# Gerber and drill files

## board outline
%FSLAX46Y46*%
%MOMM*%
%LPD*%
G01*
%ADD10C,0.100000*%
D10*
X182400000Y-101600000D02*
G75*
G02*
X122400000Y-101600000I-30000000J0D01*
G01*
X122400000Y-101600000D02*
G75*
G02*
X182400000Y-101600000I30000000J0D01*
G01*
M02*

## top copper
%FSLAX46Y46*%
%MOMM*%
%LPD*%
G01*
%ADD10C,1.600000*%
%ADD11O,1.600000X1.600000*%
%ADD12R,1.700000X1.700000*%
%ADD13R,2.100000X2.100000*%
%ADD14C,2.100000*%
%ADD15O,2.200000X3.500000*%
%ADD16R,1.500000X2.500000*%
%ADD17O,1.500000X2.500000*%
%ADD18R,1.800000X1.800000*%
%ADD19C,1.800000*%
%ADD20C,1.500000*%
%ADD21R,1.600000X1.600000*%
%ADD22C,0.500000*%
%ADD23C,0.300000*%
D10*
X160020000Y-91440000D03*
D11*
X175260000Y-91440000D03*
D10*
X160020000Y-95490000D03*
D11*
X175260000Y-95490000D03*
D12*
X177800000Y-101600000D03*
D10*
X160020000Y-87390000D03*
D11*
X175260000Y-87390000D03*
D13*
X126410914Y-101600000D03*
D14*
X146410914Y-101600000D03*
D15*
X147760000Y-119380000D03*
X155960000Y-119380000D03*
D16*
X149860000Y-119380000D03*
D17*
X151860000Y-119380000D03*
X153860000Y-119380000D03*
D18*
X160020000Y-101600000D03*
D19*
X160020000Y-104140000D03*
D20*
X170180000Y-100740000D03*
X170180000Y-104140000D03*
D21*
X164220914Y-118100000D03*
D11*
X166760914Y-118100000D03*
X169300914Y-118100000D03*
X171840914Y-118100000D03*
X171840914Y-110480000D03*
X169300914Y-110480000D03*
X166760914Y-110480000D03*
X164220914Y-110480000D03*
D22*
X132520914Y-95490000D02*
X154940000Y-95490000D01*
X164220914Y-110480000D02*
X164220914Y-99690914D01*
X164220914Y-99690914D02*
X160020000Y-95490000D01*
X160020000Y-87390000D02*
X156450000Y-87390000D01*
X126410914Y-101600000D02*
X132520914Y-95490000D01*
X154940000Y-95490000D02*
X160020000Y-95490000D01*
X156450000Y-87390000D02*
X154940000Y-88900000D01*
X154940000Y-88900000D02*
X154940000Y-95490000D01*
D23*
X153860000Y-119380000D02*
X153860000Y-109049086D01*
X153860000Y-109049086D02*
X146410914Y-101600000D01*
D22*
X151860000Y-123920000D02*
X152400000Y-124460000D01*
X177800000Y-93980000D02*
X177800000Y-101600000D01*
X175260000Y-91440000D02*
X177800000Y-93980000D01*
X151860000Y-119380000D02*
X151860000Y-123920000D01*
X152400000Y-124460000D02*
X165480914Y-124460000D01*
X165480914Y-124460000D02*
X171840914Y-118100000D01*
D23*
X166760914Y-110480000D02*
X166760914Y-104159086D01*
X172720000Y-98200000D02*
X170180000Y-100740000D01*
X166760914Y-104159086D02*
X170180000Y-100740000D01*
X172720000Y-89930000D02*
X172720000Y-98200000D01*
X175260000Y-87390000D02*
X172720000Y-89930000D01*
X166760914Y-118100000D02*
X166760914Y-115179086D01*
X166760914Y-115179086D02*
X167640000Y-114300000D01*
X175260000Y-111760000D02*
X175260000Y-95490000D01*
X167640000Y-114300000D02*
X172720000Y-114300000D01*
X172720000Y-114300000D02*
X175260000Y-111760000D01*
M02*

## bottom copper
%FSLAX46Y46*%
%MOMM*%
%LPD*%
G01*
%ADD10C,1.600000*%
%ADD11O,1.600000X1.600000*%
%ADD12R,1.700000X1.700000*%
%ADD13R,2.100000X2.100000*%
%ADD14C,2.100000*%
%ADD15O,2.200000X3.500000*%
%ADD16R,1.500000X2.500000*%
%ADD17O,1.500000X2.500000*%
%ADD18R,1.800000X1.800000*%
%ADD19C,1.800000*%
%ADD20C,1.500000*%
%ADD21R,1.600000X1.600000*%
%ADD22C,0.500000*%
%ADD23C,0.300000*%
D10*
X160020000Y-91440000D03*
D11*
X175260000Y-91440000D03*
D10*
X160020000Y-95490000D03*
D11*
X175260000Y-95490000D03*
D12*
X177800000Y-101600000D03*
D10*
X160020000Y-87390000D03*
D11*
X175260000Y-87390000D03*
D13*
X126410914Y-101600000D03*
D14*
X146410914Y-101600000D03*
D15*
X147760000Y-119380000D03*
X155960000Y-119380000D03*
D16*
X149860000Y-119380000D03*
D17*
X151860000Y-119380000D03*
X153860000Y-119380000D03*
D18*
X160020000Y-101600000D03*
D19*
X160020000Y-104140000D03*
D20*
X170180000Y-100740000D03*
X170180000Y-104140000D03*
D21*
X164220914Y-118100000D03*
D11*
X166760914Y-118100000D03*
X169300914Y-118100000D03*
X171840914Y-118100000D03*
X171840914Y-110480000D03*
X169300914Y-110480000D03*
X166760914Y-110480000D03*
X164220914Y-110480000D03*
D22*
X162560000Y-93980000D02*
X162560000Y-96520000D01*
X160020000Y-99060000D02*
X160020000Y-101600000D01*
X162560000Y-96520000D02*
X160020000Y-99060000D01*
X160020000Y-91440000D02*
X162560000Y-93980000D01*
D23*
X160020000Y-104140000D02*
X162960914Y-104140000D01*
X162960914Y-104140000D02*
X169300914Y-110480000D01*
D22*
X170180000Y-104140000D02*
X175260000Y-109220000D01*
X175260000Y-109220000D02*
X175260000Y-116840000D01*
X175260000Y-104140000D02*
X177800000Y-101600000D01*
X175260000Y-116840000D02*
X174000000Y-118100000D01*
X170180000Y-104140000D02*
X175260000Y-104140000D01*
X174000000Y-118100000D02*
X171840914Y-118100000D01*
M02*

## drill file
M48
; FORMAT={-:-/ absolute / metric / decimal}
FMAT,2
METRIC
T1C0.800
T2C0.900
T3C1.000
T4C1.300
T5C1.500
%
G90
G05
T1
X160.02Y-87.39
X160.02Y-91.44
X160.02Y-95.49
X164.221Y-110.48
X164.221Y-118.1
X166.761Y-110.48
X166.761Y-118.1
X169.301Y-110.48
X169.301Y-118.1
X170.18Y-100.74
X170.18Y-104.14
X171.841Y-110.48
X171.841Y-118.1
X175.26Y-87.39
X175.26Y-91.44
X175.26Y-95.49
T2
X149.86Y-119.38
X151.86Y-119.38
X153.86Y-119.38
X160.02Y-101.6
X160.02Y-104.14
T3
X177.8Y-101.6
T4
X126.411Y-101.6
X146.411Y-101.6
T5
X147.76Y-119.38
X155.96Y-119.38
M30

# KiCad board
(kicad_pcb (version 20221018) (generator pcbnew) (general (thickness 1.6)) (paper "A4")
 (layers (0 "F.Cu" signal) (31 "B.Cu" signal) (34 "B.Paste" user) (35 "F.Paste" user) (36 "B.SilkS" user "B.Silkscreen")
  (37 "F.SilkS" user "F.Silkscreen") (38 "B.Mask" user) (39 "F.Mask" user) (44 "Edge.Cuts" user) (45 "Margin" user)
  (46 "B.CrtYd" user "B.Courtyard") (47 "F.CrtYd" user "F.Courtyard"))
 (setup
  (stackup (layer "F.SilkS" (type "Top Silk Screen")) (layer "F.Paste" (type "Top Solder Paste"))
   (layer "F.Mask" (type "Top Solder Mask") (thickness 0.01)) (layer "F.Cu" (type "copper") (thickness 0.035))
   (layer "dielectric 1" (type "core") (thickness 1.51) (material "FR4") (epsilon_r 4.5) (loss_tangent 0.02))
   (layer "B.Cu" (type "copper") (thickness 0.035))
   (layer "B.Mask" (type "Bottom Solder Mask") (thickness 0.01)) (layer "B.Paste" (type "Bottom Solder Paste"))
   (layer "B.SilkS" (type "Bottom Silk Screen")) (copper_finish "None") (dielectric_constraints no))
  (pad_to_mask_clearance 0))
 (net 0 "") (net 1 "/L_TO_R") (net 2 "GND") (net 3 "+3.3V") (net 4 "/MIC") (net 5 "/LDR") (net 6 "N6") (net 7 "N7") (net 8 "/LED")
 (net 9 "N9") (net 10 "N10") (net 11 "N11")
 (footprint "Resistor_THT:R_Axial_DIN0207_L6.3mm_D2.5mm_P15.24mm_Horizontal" (layer "F.Cu") (at 160.02 91.44)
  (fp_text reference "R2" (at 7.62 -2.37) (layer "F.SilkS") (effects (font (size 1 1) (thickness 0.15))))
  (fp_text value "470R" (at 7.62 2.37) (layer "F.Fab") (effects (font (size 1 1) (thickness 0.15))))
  (pad "1" thru_hole circle (at 0 0) (size 1.6 1.6) (drill 0.8) (layers "*.Cu" "*.Mask") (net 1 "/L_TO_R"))
  (pad "2" thru_hole oval (at 15.24 0) (size 1.6 1.6) (drill 0.8) (layers "*.Cu" "*.Mask") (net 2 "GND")))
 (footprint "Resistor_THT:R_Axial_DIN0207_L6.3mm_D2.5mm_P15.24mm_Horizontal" (layer "F.Cu") (at 160.02 95.49)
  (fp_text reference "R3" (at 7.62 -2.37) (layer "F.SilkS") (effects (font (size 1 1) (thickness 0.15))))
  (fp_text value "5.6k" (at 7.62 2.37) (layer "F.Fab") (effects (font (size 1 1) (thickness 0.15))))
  (pad "1" thru_hole circle (at 0 0) (size 1.6 1.6) (drill 0.8) (layers "*.Cu" "*.Mask") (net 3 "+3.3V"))
  (pad "2" thru_hole oval (at 15.24 0) (size 1.6 1.6) (drill 0.8) (layers "*.Cu" "*.Mask") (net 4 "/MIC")))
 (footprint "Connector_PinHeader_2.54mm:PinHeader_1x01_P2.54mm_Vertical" (layer "F.Cu") (at 177.8 101.6 90)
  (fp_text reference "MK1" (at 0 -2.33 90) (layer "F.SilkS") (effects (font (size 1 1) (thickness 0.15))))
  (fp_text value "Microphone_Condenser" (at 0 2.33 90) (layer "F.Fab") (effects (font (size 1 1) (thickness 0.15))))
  (pad "1" thru_hole rect (at 0 0 90) (size 1.7 1.7) (drill 1) (layers "*.Cu" "*.Mask") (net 2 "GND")))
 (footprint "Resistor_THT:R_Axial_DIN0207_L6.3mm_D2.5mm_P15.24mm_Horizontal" (layer "F.Cu") (at 160.02 87.39)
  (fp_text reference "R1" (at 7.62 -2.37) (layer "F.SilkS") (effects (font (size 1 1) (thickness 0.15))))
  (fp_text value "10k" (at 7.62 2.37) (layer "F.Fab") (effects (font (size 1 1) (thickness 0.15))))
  (pad "1" thru_hole circle (at 0 0) (size 1.6 1.6) (drill 0.8) (layers "*.Cu" "*.Mask") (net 3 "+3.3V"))
  (pad "2" thru_hole oval (at 15.24 0) (size 1.6 1.6) (drill 0.8) (layers "*.Cu" "*.Mask") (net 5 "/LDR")))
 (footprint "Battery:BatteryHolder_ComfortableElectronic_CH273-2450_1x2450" (layer "F.Cu") (at 126.410914 101.6)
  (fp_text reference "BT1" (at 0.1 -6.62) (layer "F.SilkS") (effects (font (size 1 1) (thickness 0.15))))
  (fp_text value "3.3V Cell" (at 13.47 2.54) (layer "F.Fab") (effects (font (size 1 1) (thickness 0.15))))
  (pad "1" thru_hole rect (at 0 0 270) (size 2.1 2.1) (drill 1.3) (layers "*.Cu" "*.Mask") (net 3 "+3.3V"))
  (pad "2" thru_hole circle (at 20 0 270) (size 2.1 2.1) (drill 1.3) (layers "*.Cu" "*.Mask") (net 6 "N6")))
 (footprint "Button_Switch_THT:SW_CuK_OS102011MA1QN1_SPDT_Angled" (layer "F.Cu") (at 149.86 119.38)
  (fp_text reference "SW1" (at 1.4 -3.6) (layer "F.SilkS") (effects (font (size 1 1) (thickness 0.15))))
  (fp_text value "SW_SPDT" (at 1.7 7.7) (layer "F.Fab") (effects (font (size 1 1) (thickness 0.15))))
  (pad "" thru_hole oval (at -2.1 0) (size 2.2 3.5) (drill 1.5) (layers "*.Cu" "*.Mask"))
  (pad "" thru_hole oval (at 6.1 0) (size 2.2 3.5) (drill 1.5) (layers "*.Cu" "*.Mask"))
  (pad "1" thru_hole rect (at 0 0) (size 1.5 2.5) (drill 0.9) (layers "*.Cu" "*.Mask") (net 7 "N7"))
  (pad "2" thru_hole oval (at 2 0) (size 1.5 2.5) (drill 0.9) (layers "*.Cu" "*.Mask") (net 2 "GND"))
  (pad "3" thru_hole oval (at 4 0) (size 1.5 2.5) (drill 0.9) (layers "*.Cu" "*.Mask") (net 6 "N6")))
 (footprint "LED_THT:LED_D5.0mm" (layer "F.Cu") (at 160.02 101.6 -90)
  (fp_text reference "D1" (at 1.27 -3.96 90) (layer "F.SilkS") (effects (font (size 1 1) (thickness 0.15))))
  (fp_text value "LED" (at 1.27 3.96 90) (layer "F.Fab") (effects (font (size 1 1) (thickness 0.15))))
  (pad "1" thru_hole rect (at 0 0 270) (size 1.8 1.8) (drill 0.9) (layers "*.Cu" "*.Mask") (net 1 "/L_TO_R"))
  (pad "2" thru_hole circle (at 2.54 0 270) (size 1.8 1.8) (drill 0.9) (layers "*.Cu" "*.Mask") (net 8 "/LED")))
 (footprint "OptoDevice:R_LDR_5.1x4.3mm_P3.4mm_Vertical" (layer "F.Cu") (at 170.18 100.74 -90)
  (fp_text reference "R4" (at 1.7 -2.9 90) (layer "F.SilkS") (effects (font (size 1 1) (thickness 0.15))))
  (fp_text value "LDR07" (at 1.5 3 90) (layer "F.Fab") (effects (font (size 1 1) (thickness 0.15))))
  (pad "1" thru_hole circle (at 0 0 270) (size 1.5 1.5) (drill 0.8) (layers "*.Cu" "*.Mask") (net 5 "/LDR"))
  (pad "2" thru_hole circle (at 3.4 0 270) (size 1.5 1.5) (drill 0.8) (layers "*.Cu" "*.Mask") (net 2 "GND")))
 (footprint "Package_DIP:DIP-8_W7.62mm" (layer "F.Cu") (at 164.220914 118.1 90)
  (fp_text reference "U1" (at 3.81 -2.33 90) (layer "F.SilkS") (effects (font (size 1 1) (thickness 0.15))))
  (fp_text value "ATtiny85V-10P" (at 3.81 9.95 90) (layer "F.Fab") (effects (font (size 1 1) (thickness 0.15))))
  (pad "1" thru_hole rect (at 0 0 90) (size 1.6 1.6) (drill 0.8) (layers "*.Cu" "*.Mask") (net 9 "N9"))
  (pad "2" thru_hole oval (at 0 2.54 90) (size 1.6 1.6) (drill 0.8) (layers "*.Cu" "*.Mask") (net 4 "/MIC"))
  (pad "3" thru_hole oval (at 0 5.08 90) (size 1.6 1.6) (drill 0.8) (layers "*.Cu" "*.Mask") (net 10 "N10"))
  (pad "4" thru_hole oval (at 0 7.62 90) (size 1.6 1.6) (drill 0.8) (layers "*.Cu" "*.Mask") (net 2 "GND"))
  (pad "5" thru_hole oval (at 7.62 7.62 90) (size 1.6 1.6) (drill 0.8) (layers "*.Cu" "*.Mask") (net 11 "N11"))
  (pad "6" thru_hole oval (at 7.62 5.08 90) (size 1.6 1.6) (drill 0.8) (layers "*.Cu" "*.Mask") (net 8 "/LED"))
  (pad "7" thru_hole oval (at 7.62 2.54 90) (size 1.6 1.6) (drill 0.8) (layers "*.Cu" "*.Mask") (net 5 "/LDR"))
  (pad "8" thru_hole oval (at 7.62 0 90) (size 1.6 1.6) (drill 0.8) (layers "*.Cu" "*.Mask") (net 3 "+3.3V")))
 (gr_circle locked (center 152.4 101.6) (end 182.4 101.6) (stroke (width 0.1) (type solid)) (fill none) (layer "Edge.Cuts"))
 (segment (start 132.520914 95.49) (end 154.94 95.49) (width 0.5) (layer "F.Cu") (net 3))
 (segment (start 164.220914 110.48) (end 164.220914 99.690914) (width 0.5) (layer "F.Cu") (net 3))
 (segment (start 164.220914 99.690914) (end 160.02 95.49) (width 0.5) (layer "F.Cu") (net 3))
 (segment (start 160.02 87.39) (end 156.45 87.39) (width 0.5) (layer "F.Cu") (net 3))
 (segment (start 126.410914 101.6) (end 132.520914 95.49) (width 0.5) (layer "F.Cu") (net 3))
 (segment (start 154.94 95.49) (end 160.02 95.49) (width 0.5) (layer "F.Cu") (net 3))
 (segment (start 156.45 87.39) (end 154.94 88.9) (width 0.5) (layer "F.Cu") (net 3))
 (segment (start 154.94 88.9) (end 154.94 95.49) (width 0.5) (layer "F.Cu") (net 3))
 (segment (start 153.86 119.38) (end 153.86 109.049086) (width 0.3) (layer "F.Cu") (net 6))
 (segment (start 153.86 109.049086) (end 146.410914 101.6) (width 0.3) (layer "F.Cu") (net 6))
 (segment (start 162.56 93.98) (end 162.56 96.52) (width 0.5) (layer "B.Cu") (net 1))
 (segment (start 160.02 99.06) (end 160.02 101.6) (width 0.5) (layer "B.Cu") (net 1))
 (segment (start 162.56 96.52) (end 160.02 99.06) (width 0.5) (layer "B.Cu") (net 1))
 (segment (start 160.02 91.44) (end 162.56 93.98) (width 0.5) (layer "B.Cu") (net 1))
 (segment (start 160.02 104.14) (end 162.960914 104.14) (width 0.3) (layer "B.Cu") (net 8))
 (segment (start 162.960914 104.14) (end 169.300914 110.48) (width 0.3) (layer "B.Cu") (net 8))
 (segment (start 151.86 123.92) (end 152.4 124.46) (width 0.5) (layer "F.Cu") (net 2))
 (segment (start 177.8 93.98) (end 177.8 101.6) (width 0.5) (layer "F.Cu") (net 2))
 (segment (start 175.26 91.44) (end 177.8 93.98) (width 0.5) (layer "F.Cu") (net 2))
 (segment (start 151.86 119.38) (end 151.86 123.92) (width 0.5) (layer "F.Cu") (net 2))
 (segment (start 152.4 124.46) (end 165.480914 124.46) (width 0.5) (layer "F.Cu") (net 2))
 (segment (start 165.480914 124.46) (end 171.840914 118.1) (width 0.5) (layer "F.Cu") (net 2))
 (segment (start 170.18 104.14) (end 175.26 109.22) (width 0.5) (layer "B.Cu") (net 2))
 (segment (start 175.26 109.22) (end 175.26 116.84) (width 0.5) (layer "B.Cu") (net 2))
 (segment (start 175.26 104.14) (end 177.8 101.6) (width 0.5) (layer "B.Cu") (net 2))
 (segment (start 175.26 116.84) (end 174 118.1) (width 0.5) (layer "B.Cu") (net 2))
 (segment (start 170.18 104.14) (end 175.26 104.14) (width 0.5) (layer "B.Cu") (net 2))
 (segment (start 174 118.1) (end 171.840914 118.1) (width 0.5) (layer "B.Cu") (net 2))
 (segment (start 166.760914 110.48) (end 166.760914 104.159086) (width 0.3) (layer "F.Cu") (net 5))
 (segment (start 172.72 98.2) (end 170.18 100.74) (width 0.3) (layer "F.Cu") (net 5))
 (segment (start 166.760914 104.159086) (end 170.18 100.74) (width 0.3) (layer "F.Cu") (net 5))
 (segment (start 172.72 89.93) (end 172.72 98.2) (width 0.3) (layer "F.Cu") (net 5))
 (segment (start 175.26 87.39) (end 172.72 89.93) (width 0.3) (layer "F.Cu") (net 5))
 (segment (start 166.760914 118.1) (end 166.760914 115.179086) (width 0.3) (layer "F.Cu") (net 4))
 (segment (start 166.760914 115.179086) (end 167.64 114.3) (width 0.3) (layer "F.Cu") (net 4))
 (segment (start 175.26 111.76) (end 175.26 95.49) (width 0.3) (layer "F.Cu") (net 4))
 (segment (start 167.64 114.3) (end 172.72 114.3) (width 0.3) (layer "F.Cu") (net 4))
 (segment (start 172.72 114.3) (end 175.26 111.76) (width 0.3) (layer "F.Cu") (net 4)))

